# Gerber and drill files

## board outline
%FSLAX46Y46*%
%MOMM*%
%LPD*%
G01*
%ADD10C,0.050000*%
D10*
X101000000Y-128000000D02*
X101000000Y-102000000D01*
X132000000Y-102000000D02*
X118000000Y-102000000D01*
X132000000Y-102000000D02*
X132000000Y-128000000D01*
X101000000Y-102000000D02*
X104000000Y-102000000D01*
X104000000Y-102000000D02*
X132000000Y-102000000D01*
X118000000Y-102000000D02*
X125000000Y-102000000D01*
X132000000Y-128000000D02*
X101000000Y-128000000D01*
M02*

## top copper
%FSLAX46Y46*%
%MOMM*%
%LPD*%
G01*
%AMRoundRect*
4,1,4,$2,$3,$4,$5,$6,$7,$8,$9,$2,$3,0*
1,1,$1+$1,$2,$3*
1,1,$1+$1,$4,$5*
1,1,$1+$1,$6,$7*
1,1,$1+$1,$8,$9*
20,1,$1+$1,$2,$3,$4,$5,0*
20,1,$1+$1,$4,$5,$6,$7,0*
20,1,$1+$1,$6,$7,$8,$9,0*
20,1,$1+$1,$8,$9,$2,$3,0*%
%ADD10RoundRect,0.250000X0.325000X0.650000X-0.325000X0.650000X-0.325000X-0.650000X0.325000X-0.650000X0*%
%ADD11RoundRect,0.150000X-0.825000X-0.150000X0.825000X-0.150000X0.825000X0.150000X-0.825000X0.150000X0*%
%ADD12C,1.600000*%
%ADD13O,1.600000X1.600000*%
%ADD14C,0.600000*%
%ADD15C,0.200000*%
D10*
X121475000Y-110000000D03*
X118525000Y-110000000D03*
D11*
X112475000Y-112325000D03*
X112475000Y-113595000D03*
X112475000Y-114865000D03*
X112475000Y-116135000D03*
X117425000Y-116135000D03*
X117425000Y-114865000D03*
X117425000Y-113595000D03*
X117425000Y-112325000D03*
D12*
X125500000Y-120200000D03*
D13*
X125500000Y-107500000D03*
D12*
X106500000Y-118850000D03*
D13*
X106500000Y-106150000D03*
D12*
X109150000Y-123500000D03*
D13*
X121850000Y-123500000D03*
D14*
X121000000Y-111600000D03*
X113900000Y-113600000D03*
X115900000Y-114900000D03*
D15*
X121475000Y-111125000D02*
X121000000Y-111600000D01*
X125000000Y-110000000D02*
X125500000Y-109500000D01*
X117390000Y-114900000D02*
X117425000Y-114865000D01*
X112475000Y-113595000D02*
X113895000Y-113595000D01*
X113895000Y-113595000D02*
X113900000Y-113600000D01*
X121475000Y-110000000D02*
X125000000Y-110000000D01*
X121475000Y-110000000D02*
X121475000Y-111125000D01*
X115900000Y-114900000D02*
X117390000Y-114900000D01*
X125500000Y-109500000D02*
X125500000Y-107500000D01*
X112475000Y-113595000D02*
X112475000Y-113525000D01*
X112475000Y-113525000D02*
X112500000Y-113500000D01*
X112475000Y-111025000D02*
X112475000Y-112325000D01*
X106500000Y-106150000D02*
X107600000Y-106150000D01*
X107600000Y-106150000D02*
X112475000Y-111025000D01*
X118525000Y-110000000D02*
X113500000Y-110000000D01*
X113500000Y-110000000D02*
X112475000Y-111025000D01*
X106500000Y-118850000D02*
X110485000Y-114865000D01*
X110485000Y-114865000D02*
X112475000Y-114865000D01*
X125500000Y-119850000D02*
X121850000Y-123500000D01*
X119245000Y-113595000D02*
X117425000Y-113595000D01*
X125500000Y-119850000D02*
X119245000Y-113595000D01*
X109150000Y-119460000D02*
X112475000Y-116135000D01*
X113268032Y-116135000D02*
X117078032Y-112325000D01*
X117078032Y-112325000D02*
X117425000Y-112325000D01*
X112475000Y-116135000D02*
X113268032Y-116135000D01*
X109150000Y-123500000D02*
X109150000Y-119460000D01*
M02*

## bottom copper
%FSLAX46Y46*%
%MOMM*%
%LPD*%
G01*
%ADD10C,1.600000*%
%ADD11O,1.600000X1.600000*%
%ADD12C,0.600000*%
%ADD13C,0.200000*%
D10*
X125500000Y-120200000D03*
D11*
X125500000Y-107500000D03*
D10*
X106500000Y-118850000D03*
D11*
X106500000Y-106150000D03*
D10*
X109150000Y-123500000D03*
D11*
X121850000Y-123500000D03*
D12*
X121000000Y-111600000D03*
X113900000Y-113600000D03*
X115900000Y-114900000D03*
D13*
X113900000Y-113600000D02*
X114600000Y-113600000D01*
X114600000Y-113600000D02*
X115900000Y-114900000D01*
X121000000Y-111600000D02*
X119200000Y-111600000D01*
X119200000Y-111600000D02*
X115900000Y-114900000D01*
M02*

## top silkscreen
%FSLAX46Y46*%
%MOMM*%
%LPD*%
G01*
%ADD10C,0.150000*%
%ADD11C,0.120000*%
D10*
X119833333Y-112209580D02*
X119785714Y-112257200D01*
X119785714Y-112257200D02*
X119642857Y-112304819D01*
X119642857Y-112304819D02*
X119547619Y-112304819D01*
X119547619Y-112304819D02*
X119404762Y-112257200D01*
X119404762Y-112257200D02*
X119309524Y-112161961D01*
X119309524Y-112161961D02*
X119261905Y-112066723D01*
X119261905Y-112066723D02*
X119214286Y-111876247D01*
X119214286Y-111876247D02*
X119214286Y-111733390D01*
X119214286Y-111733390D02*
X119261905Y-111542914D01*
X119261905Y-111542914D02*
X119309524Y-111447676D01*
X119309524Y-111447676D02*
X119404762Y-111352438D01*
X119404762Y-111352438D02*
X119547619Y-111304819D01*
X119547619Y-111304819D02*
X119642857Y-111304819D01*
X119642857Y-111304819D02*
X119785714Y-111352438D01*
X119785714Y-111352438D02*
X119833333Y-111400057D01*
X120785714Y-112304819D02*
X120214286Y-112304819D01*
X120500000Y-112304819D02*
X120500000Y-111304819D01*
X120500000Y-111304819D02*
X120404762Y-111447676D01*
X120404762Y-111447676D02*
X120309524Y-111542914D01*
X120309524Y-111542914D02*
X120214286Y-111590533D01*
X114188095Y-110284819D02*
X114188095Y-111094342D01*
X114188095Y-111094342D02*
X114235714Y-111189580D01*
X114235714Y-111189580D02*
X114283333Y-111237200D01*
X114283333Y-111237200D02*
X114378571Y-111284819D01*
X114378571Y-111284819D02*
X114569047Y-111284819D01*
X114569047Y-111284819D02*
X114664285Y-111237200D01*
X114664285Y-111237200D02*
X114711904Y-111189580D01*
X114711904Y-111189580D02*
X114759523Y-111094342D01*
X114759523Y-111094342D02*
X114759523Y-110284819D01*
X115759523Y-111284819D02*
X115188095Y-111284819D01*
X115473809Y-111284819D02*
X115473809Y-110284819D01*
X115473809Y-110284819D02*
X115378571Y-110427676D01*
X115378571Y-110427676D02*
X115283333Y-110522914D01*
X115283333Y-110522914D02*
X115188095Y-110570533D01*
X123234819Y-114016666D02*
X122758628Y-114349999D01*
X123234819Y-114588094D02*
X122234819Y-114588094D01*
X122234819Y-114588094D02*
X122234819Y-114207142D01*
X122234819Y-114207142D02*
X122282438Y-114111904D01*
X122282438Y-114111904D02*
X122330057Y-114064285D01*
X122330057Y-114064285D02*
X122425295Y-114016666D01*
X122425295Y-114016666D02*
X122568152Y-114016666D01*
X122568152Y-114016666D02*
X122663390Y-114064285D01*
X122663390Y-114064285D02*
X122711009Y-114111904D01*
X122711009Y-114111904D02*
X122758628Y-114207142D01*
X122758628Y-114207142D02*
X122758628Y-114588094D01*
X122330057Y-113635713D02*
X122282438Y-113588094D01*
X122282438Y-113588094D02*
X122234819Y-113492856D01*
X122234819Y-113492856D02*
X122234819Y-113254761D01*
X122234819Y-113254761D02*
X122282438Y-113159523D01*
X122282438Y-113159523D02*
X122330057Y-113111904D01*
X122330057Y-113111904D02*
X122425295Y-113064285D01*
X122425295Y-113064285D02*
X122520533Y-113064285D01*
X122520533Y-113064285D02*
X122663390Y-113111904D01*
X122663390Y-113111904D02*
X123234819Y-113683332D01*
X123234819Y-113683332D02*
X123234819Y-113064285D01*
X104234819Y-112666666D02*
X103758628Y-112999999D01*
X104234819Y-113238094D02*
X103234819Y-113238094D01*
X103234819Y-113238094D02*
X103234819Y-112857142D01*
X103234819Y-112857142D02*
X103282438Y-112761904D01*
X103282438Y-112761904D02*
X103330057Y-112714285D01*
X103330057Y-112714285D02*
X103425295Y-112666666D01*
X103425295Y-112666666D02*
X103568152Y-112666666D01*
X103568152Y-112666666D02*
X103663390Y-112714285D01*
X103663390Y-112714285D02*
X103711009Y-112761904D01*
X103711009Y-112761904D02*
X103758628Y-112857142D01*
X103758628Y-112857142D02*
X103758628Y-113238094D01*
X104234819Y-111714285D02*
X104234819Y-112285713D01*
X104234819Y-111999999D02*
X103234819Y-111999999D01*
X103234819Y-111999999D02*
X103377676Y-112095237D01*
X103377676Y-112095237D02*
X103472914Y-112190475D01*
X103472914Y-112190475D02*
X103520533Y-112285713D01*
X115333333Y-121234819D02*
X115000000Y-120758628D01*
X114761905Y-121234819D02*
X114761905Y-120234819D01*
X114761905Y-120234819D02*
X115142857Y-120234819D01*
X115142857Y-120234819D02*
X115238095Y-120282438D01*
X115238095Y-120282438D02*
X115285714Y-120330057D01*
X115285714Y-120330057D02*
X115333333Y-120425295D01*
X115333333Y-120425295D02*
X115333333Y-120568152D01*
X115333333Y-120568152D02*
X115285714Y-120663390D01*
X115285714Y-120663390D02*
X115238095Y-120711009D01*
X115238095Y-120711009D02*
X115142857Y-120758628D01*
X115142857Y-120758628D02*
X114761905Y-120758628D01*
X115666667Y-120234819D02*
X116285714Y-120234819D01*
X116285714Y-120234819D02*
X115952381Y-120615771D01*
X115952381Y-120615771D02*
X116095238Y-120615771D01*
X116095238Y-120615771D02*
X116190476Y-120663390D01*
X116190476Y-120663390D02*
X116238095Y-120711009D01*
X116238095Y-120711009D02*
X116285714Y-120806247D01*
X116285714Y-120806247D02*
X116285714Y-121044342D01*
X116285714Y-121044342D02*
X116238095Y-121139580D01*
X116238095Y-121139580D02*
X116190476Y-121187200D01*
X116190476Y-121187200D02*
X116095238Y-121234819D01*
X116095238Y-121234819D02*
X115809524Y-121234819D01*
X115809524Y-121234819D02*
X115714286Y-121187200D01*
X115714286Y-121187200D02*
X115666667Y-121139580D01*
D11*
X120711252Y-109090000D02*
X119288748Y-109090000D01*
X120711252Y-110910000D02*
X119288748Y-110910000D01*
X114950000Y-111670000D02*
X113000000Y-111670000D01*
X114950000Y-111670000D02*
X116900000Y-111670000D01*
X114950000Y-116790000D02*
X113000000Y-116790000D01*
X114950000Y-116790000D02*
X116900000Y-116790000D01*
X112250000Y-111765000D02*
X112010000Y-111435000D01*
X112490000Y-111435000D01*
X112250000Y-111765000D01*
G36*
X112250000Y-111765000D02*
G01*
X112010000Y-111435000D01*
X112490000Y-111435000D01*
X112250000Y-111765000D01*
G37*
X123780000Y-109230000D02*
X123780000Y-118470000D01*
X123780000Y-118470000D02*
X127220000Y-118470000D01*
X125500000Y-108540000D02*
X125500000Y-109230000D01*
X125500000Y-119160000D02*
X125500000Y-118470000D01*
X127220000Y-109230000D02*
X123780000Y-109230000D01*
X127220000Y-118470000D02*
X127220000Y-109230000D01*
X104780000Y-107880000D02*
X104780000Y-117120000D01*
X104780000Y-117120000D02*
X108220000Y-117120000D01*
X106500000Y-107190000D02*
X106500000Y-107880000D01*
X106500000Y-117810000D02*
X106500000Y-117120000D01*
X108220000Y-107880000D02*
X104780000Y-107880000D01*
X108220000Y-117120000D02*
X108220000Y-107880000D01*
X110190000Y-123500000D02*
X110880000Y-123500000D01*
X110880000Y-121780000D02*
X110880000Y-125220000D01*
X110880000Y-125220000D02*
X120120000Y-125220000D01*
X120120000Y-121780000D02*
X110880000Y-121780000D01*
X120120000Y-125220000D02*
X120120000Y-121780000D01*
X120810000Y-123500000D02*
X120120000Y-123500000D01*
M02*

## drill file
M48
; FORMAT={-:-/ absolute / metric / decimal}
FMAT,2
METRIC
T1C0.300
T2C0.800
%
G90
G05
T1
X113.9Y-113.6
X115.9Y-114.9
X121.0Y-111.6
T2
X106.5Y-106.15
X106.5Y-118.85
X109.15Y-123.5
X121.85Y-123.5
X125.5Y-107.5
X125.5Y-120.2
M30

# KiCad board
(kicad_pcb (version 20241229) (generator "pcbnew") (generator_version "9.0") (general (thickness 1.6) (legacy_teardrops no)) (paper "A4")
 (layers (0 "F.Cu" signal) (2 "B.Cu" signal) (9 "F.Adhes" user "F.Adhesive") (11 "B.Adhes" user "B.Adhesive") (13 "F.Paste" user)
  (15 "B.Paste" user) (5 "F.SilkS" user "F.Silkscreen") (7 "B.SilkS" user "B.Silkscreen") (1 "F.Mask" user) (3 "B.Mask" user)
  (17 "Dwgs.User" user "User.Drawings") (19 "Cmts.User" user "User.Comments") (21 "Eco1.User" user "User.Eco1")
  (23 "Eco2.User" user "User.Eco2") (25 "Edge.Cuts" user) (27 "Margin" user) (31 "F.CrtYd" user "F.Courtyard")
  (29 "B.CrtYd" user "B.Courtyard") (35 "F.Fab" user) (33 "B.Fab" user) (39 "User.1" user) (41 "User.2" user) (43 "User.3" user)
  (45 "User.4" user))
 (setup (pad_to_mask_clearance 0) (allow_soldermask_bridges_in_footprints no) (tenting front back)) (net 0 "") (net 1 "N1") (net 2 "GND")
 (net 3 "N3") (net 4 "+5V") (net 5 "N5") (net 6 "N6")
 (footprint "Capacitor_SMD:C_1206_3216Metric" (layer "F.Cu") (at 120 110 180)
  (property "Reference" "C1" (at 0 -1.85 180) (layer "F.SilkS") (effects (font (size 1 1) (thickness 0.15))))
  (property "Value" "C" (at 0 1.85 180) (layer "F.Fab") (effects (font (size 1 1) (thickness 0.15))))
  (fp_line (start -0.711252 0.91) (end 0.711252 0.91) (stroke (width 0.12) (type solid)) (layer "F.SilkS"))
  (fp_line (start -0.711252 -0.91) (end 0.711252 -0.91) (stroke (width 0.12) (type solid)) (layer "F.SilkS"))
  (pad "1" smd roundrect (at -1.475 0 180) (size 1.15 1.8) (layers "F.Cu" "F.Mask" "F.Paste") (roundrect_rratio 0.217391) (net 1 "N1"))
  (pad "2" smd roundrect (at 1.475 0 180) (size 1.15 1.8) (layers "F.Cu" "F.Mask" "F.Paste") (roundrect_rratio 0.217391) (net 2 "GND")))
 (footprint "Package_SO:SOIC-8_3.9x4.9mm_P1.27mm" (layer "F.Cu") (at 114.95 114.23)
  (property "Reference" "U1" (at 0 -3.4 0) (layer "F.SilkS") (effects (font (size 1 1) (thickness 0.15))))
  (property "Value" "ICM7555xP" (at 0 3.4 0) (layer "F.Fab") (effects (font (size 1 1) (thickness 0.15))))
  (fp_line (start 0 -2.56) (end -1.95 -2.56) (stroke (width 0.12) (type solid)) (layer "F.SilkS"))
  (fp_line (start 0 -2.56) (end 1.95 -2.56) (stroke (width 0.12) (type solid)) (layer "F.SilkS"))
  (fp_line (start 0 2.56) (end -1.95 2.56) (stroke (width 0.12) (type solid)) (layer "F.SilkS"))
  (fp_line (start 0 2.56) (end 1.95 2.56) (stroke (width 0.12) (type solid)) (layer "F.SilkS"))
  (fp_poly
   (pts (xy -2.7 -2.465) (xy -2.94 -2.795) (xy -2.46 -2.795) (xy -2.7 -2.465)) (stroke (width 0.12) (type solid)) (fill yes)
   (layer "F.SilkS"))
  (pad "1" smd roundrect (at -2.475 -1.905) (size 1.95 0.6) (layers "F.Cu" "F.Mask" "F.Paste") (roundrect_rratio 0.25) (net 2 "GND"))
  (pad "2" smd roundrect (at -2.475 -0.635) (size 1.95 0.6) (layers "F.Cu" "F.Mask" "F.Paste") (roundrect_rratio 0.25) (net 1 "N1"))
  (pad "3" smd roundrect (at -2.475 0.635) (size 1.95 0.6) (layers "F.Cu" "F.Mask" "F.Paste") (roundrect_rratio 0.25) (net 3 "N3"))
  (pad "4" smd roundrect (at -2.475 1.905) (size 1.95 0.6) (layers "F.Cu" "F.Mask" "F.Paste") (roundrect_rratio 0.25) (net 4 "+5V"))
  (pad "5" smd roundrect (at 2.475 1.905) (size 1.95 0.6) (layers "F.Cu" "F.Mask" "F.Paste") (roundrect_rratio 0.25) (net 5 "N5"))
  (pad "6" smd roundrect (at 2.475 0.635) (size 1.95 0.6) (layers "F.Cu" "F.Mask" "F.Paste") (roundrect_rratio 0.25) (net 1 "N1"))
  (pad "7" smd roundrect (at 2.475 -0.635) (size 1.95 0.6) (layers "F.Cu" "F.Mask" "F.Paste") (roundrect_rratio 0.25) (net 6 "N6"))
  (pad "8" smd roundrect (at 2.475 -1.905) (size 1.95 0.6) (layers "F.Cu" "F.Mask" "F.Paste") (roundrect_rratio 0.25) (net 4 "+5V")))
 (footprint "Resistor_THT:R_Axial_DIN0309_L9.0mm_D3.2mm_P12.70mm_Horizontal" (layer "F.Cu") (at 125.5 120.2 90)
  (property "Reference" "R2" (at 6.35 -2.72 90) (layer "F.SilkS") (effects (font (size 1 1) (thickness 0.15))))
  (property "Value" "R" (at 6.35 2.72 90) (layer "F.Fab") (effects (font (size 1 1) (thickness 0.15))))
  (fp_line (start 10.97 -1.72) (end 1.73 -1.72) (stroke (width 0.12) (type solid)) (layer "F.SilkS"))
  (fp_line (start 1.73 -1.72) (end 1.73 1.72) (stroke (width 0.12) (type solid)) (layer "F.SilkS"))
  (fp_line (start 11.66 0) (end 10.97 0) (stroke (width 0.12) (type solid)) (layer "F.SilkS"))
  (fp_line (start 1.04 0) (end 1.73 0) (stroke (width 0.12) (type solid)) (layer "F.SilkS"))
  (fp_line (start 10.97 1.72) (end 10.97 -1.72) (stroke (width 0.12) (type solid)) (layer "F.SilkS"))
  (fp_line (start 1.73 1.72) (end 10.97 1.72) (stroke (width 0.12) (type solid)) (layer "F.SilkS"))
  (pad "1" thru_hole circle (at 0 0 90) (size 1.6 1.6) (drill 0.8) (layers "*.Cu" "*.Mask") (remove_unused_layers no) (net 6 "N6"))
  (pad "2" thru_hole oval (at 12.7 0 90) (size 1.6 1.6) (drill 0.8) (layers "*.Cu" "*.Mask") (remove_unused_layers no) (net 1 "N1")))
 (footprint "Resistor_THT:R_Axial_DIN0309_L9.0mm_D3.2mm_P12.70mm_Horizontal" (layer "F.Cu") (at 106.5 118.85 90)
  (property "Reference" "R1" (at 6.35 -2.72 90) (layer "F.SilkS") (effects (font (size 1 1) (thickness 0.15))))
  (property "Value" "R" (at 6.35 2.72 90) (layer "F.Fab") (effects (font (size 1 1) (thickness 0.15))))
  (fp_line (start 10.97 -1.72) (end 1.73 -1.72) (stroke (width 0.12) (type solid)) (layer "F.SilkS"))
  (fp_line (start 1.73 -1.72) (end 1.73 1.72) (stroke (width 0.12) (type solid)) (layer "F.SilkS"))
  (fp_line (start 11.66 0) (end 10.97 0) (stroke (width 0.12) (type solid)) (layer "F.SilkS"))
  (fp_line (start 1.04 0) (end 1.73 0) (stroke (width 0.12) (type solid)) (layer "F.SilkS"))
  (fp_line (start 10.97 1.72) (end 10.97 -1.72) (stroke (width 0.12) (type solid)) (layer "F.SilkS"))
  (fp_line (start 1.73 1.72) (end 10.97 1.72) (stroke (width 0.12) (type solid)) (layer "F.SilkS"))
  (pad "1" thru_hole circle (at 0 0 90) (size 1.6 1.6) (drill 0.8) (layers "*.Cu" "*.Mask") (remove_unused_layers no) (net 3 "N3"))
  (pad "2" thru_hole oval (at 12.7 0 90) (size 1.6 1.6) (drill 0.8) (layers "*.Cu" "*.Mask") (remove_unused_layers no) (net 2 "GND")))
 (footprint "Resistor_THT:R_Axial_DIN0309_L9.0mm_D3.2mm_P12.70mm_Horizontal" (layer "F.Cu") (at 109.15 123.5)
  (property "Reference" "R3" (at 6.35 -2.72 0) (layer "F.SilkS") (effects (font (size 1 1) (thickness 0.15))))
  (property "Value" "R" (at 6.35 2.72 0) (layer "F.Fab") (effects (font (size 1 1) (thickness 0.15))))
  (fp_line (start 1.04 0) (end 1.73 0) (stroke (width 0.12) (type solid)) (layer "F.SilkS"))
  (fp_line (start 1.73 -1.72) (end 1.73 1.72) (stroke (width 0.12) (type solid)) (layer "F.SilkS"))
  (fp_line (start 1.73 1.72) (end 10.97 1.72) (stroke (width 0.12) (type solid)) (layer "F.SilkS"))
  (fp_line (start 10.97 -1.72) (end 1.73 -1.72) (stroke (width 0.12) (type solid)) (layer "F.SilkS"))
  (fp_line (start 10.97 1.72) (end 10.97 -1.72) (stroke (width 0.12) (type solid)) (layer "F.SilkS"))
  (fp_line (start 11.66 0) (end 10.97 0) (stroke (width 0.12) (type solid)) (layer "F.SilkS"))
  (pad "1" thru_hole circle (at 0 0) (size 1.6 1.6) (drill 0.8) (layers "*.Cu" "*.Mask") (remove_unused_layers no) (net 4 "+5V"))
  (pad "2" thru_hole oval (at 12.7 0) (size 1.6 1.6) (drill 0.8) (layers "*.Cu" "*.Mask") (remove_unused_layers no) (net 6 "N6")))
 (gr_line (start 101 128) (end 101 102) (stroke (width 0.05) (type default)) (layer "Edge.Cuts"))
 (gr_line (start 132 102) (end 118 102) (stroke (width 0.05) (type default)) (layer "Edge.Cuts"))
 (gr_line (start 132 102) (end 132 128) (stroke (width 0.05) (type default)) (layer "Edge.Cuts"))
 (gr_line (start 101 102) (end 104 102) (stroke (width 0.05) (type default)) (layer "Edge.Cuts"))
 (gr_line (start 104 102) (end 132 102) (stroke (width 0.05) (type default)) (layer "Edge.Cuts"))
 (gr_line (start 118 102) (end 125 102) (stroke (width 0.05) (type default)) (layer "Edge.Cuts"))
 (gr_line (start 132 128) (end 101 128) (stroke (width 0.05) (type default)) (layer "Edge.Cuts"))
 (segment (start 121.475 111.125) (end 121 111.6) (width 0.2) (layer "F.Cu") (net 1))
 (segment (start 125 110) (end 125.5 109.5) (width 0.2) (layer "F.Cu") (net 1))
 (segment (start 117.39 114.9) (end 117.425 114.865) (width 0.2) (layer "F.Cu") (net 1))
 (segment (start 112.475 113.595) (end 113.895 113.595) (width 0.2) (layer "F.Cu") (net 1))
 (segment (start 113.895 113.595) (end 113.9 113.6) (width 0.2) (layer "F.Cu") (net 1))
 (segment (start 121.475 110) (end 125 110) (width 0.2) (layer "F.Cu") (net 1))
 (segment (start 121.475 110) (end 121.475 111.125) (width 0.2) (layer "F.Cu") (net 1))
 (segment (start 115.9 114.9) (end 117.39 114.9) (width 0.2) (layer "F.Cu") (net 1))
 (segment (start 125.5 109.5) (end 125.5 107.5) (width 0.2) (layer "F.Cu") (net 1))
 (segment (start 112.475 113.595) (end 112.475 113.525) (width 0.2) (layer "F.Cu") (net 1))
 (segment (start 112.475 113.525) (end 112.5 113.5) (width 0.2) (layer "F.Cu") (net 1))
 (via (at 121 111.6) (size 0.6) (drill 0.3) (layers "F.Cu" "B.Cu") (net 1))
 (via (at 113.9 113.6) (size 0.6) (drill 0.3) (layers "F.Cu" "B.Cu") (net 1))
 (via (at 115.9 114.9) (size 0.6) (drill 0.3) (layers "F.Cu" "B.Cu") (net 1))
 (segment (start 113.9 113.6) (end 114.6 113.6) (width 0.2) (layer "B.Cu") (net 1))
 (segment (start 114.6 113.6) (end 115.9 114.9) (width 0.2) (layer "B.Cu") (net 1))
 (segment (start 121 111.6) (end 119.2 111.6) (width 0.2) (layer "B.Cu") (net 1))
 (segment (start 119.2 111.6) (end 115.9 114.9) (width 0.2) (layer "B.Cu") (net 1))
 (segment (start 112.475 111.025) (end 112.475 112.325) (width 0.2) (layer "F.Cu") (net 2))
 (segment (start 106.5 106.15) (end 107.6 106.15) (width 0.2) (layer "F.Cu") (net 2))
 (segment (start 107.6 106.15) (end 112.475 111.025) (width 0.2) (layer "F.Cu") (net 2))
 (segment (start 118.525 110) (end 113.5 110) (width 0.2) (layer "F.Cu") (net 2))
 (segment (start 113.5 110) (end 112.475 111.025) (width 0.2) (layer "F.Cu") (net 2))
 (segment (start 106.5 118.85) (end 110.485 114.865) (width 0.2) (layer "F.Cu") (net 3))
 (segment (start 110.485 114.865) (end 112.475 114.865) (width 0.2) (layer "F.Cu") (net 3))
 (segment (start 125.5 119.85) (end 121.85 123.5) (width 0.2) (layer "F.Cu") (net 6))
 (segment (start 119.245 113.595) (end 117.425 113.595) (width 0.2) (layer "F.Cu") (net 6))
 (segment (start 125.5 119.85) (end 119.245 113.595) (width 0.2) (layer "F.Cu") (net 6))
 (segment (start 109.15 119.46) (end 112.475 116.135) (width 0.2) (layer "F.Cu") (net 4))
 (segment (start 113.268032 116.135) (end 117.078032 112.325) (width 0.2) (layer "F.Cu") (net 4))
 (segment (start 117.078032 112.325) (end 117.425 112.325) (width 0.2) (layer "F.Cu") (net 4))
 (segment (start 112.475 116.135) (end 113.268032 116.135) (width 0.2) (layer "F.Cu") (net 4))
 (segment (start 109.15 123.5) (end 109.15 119.46) (width 0.2) (layer "F.Cu") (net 4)))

